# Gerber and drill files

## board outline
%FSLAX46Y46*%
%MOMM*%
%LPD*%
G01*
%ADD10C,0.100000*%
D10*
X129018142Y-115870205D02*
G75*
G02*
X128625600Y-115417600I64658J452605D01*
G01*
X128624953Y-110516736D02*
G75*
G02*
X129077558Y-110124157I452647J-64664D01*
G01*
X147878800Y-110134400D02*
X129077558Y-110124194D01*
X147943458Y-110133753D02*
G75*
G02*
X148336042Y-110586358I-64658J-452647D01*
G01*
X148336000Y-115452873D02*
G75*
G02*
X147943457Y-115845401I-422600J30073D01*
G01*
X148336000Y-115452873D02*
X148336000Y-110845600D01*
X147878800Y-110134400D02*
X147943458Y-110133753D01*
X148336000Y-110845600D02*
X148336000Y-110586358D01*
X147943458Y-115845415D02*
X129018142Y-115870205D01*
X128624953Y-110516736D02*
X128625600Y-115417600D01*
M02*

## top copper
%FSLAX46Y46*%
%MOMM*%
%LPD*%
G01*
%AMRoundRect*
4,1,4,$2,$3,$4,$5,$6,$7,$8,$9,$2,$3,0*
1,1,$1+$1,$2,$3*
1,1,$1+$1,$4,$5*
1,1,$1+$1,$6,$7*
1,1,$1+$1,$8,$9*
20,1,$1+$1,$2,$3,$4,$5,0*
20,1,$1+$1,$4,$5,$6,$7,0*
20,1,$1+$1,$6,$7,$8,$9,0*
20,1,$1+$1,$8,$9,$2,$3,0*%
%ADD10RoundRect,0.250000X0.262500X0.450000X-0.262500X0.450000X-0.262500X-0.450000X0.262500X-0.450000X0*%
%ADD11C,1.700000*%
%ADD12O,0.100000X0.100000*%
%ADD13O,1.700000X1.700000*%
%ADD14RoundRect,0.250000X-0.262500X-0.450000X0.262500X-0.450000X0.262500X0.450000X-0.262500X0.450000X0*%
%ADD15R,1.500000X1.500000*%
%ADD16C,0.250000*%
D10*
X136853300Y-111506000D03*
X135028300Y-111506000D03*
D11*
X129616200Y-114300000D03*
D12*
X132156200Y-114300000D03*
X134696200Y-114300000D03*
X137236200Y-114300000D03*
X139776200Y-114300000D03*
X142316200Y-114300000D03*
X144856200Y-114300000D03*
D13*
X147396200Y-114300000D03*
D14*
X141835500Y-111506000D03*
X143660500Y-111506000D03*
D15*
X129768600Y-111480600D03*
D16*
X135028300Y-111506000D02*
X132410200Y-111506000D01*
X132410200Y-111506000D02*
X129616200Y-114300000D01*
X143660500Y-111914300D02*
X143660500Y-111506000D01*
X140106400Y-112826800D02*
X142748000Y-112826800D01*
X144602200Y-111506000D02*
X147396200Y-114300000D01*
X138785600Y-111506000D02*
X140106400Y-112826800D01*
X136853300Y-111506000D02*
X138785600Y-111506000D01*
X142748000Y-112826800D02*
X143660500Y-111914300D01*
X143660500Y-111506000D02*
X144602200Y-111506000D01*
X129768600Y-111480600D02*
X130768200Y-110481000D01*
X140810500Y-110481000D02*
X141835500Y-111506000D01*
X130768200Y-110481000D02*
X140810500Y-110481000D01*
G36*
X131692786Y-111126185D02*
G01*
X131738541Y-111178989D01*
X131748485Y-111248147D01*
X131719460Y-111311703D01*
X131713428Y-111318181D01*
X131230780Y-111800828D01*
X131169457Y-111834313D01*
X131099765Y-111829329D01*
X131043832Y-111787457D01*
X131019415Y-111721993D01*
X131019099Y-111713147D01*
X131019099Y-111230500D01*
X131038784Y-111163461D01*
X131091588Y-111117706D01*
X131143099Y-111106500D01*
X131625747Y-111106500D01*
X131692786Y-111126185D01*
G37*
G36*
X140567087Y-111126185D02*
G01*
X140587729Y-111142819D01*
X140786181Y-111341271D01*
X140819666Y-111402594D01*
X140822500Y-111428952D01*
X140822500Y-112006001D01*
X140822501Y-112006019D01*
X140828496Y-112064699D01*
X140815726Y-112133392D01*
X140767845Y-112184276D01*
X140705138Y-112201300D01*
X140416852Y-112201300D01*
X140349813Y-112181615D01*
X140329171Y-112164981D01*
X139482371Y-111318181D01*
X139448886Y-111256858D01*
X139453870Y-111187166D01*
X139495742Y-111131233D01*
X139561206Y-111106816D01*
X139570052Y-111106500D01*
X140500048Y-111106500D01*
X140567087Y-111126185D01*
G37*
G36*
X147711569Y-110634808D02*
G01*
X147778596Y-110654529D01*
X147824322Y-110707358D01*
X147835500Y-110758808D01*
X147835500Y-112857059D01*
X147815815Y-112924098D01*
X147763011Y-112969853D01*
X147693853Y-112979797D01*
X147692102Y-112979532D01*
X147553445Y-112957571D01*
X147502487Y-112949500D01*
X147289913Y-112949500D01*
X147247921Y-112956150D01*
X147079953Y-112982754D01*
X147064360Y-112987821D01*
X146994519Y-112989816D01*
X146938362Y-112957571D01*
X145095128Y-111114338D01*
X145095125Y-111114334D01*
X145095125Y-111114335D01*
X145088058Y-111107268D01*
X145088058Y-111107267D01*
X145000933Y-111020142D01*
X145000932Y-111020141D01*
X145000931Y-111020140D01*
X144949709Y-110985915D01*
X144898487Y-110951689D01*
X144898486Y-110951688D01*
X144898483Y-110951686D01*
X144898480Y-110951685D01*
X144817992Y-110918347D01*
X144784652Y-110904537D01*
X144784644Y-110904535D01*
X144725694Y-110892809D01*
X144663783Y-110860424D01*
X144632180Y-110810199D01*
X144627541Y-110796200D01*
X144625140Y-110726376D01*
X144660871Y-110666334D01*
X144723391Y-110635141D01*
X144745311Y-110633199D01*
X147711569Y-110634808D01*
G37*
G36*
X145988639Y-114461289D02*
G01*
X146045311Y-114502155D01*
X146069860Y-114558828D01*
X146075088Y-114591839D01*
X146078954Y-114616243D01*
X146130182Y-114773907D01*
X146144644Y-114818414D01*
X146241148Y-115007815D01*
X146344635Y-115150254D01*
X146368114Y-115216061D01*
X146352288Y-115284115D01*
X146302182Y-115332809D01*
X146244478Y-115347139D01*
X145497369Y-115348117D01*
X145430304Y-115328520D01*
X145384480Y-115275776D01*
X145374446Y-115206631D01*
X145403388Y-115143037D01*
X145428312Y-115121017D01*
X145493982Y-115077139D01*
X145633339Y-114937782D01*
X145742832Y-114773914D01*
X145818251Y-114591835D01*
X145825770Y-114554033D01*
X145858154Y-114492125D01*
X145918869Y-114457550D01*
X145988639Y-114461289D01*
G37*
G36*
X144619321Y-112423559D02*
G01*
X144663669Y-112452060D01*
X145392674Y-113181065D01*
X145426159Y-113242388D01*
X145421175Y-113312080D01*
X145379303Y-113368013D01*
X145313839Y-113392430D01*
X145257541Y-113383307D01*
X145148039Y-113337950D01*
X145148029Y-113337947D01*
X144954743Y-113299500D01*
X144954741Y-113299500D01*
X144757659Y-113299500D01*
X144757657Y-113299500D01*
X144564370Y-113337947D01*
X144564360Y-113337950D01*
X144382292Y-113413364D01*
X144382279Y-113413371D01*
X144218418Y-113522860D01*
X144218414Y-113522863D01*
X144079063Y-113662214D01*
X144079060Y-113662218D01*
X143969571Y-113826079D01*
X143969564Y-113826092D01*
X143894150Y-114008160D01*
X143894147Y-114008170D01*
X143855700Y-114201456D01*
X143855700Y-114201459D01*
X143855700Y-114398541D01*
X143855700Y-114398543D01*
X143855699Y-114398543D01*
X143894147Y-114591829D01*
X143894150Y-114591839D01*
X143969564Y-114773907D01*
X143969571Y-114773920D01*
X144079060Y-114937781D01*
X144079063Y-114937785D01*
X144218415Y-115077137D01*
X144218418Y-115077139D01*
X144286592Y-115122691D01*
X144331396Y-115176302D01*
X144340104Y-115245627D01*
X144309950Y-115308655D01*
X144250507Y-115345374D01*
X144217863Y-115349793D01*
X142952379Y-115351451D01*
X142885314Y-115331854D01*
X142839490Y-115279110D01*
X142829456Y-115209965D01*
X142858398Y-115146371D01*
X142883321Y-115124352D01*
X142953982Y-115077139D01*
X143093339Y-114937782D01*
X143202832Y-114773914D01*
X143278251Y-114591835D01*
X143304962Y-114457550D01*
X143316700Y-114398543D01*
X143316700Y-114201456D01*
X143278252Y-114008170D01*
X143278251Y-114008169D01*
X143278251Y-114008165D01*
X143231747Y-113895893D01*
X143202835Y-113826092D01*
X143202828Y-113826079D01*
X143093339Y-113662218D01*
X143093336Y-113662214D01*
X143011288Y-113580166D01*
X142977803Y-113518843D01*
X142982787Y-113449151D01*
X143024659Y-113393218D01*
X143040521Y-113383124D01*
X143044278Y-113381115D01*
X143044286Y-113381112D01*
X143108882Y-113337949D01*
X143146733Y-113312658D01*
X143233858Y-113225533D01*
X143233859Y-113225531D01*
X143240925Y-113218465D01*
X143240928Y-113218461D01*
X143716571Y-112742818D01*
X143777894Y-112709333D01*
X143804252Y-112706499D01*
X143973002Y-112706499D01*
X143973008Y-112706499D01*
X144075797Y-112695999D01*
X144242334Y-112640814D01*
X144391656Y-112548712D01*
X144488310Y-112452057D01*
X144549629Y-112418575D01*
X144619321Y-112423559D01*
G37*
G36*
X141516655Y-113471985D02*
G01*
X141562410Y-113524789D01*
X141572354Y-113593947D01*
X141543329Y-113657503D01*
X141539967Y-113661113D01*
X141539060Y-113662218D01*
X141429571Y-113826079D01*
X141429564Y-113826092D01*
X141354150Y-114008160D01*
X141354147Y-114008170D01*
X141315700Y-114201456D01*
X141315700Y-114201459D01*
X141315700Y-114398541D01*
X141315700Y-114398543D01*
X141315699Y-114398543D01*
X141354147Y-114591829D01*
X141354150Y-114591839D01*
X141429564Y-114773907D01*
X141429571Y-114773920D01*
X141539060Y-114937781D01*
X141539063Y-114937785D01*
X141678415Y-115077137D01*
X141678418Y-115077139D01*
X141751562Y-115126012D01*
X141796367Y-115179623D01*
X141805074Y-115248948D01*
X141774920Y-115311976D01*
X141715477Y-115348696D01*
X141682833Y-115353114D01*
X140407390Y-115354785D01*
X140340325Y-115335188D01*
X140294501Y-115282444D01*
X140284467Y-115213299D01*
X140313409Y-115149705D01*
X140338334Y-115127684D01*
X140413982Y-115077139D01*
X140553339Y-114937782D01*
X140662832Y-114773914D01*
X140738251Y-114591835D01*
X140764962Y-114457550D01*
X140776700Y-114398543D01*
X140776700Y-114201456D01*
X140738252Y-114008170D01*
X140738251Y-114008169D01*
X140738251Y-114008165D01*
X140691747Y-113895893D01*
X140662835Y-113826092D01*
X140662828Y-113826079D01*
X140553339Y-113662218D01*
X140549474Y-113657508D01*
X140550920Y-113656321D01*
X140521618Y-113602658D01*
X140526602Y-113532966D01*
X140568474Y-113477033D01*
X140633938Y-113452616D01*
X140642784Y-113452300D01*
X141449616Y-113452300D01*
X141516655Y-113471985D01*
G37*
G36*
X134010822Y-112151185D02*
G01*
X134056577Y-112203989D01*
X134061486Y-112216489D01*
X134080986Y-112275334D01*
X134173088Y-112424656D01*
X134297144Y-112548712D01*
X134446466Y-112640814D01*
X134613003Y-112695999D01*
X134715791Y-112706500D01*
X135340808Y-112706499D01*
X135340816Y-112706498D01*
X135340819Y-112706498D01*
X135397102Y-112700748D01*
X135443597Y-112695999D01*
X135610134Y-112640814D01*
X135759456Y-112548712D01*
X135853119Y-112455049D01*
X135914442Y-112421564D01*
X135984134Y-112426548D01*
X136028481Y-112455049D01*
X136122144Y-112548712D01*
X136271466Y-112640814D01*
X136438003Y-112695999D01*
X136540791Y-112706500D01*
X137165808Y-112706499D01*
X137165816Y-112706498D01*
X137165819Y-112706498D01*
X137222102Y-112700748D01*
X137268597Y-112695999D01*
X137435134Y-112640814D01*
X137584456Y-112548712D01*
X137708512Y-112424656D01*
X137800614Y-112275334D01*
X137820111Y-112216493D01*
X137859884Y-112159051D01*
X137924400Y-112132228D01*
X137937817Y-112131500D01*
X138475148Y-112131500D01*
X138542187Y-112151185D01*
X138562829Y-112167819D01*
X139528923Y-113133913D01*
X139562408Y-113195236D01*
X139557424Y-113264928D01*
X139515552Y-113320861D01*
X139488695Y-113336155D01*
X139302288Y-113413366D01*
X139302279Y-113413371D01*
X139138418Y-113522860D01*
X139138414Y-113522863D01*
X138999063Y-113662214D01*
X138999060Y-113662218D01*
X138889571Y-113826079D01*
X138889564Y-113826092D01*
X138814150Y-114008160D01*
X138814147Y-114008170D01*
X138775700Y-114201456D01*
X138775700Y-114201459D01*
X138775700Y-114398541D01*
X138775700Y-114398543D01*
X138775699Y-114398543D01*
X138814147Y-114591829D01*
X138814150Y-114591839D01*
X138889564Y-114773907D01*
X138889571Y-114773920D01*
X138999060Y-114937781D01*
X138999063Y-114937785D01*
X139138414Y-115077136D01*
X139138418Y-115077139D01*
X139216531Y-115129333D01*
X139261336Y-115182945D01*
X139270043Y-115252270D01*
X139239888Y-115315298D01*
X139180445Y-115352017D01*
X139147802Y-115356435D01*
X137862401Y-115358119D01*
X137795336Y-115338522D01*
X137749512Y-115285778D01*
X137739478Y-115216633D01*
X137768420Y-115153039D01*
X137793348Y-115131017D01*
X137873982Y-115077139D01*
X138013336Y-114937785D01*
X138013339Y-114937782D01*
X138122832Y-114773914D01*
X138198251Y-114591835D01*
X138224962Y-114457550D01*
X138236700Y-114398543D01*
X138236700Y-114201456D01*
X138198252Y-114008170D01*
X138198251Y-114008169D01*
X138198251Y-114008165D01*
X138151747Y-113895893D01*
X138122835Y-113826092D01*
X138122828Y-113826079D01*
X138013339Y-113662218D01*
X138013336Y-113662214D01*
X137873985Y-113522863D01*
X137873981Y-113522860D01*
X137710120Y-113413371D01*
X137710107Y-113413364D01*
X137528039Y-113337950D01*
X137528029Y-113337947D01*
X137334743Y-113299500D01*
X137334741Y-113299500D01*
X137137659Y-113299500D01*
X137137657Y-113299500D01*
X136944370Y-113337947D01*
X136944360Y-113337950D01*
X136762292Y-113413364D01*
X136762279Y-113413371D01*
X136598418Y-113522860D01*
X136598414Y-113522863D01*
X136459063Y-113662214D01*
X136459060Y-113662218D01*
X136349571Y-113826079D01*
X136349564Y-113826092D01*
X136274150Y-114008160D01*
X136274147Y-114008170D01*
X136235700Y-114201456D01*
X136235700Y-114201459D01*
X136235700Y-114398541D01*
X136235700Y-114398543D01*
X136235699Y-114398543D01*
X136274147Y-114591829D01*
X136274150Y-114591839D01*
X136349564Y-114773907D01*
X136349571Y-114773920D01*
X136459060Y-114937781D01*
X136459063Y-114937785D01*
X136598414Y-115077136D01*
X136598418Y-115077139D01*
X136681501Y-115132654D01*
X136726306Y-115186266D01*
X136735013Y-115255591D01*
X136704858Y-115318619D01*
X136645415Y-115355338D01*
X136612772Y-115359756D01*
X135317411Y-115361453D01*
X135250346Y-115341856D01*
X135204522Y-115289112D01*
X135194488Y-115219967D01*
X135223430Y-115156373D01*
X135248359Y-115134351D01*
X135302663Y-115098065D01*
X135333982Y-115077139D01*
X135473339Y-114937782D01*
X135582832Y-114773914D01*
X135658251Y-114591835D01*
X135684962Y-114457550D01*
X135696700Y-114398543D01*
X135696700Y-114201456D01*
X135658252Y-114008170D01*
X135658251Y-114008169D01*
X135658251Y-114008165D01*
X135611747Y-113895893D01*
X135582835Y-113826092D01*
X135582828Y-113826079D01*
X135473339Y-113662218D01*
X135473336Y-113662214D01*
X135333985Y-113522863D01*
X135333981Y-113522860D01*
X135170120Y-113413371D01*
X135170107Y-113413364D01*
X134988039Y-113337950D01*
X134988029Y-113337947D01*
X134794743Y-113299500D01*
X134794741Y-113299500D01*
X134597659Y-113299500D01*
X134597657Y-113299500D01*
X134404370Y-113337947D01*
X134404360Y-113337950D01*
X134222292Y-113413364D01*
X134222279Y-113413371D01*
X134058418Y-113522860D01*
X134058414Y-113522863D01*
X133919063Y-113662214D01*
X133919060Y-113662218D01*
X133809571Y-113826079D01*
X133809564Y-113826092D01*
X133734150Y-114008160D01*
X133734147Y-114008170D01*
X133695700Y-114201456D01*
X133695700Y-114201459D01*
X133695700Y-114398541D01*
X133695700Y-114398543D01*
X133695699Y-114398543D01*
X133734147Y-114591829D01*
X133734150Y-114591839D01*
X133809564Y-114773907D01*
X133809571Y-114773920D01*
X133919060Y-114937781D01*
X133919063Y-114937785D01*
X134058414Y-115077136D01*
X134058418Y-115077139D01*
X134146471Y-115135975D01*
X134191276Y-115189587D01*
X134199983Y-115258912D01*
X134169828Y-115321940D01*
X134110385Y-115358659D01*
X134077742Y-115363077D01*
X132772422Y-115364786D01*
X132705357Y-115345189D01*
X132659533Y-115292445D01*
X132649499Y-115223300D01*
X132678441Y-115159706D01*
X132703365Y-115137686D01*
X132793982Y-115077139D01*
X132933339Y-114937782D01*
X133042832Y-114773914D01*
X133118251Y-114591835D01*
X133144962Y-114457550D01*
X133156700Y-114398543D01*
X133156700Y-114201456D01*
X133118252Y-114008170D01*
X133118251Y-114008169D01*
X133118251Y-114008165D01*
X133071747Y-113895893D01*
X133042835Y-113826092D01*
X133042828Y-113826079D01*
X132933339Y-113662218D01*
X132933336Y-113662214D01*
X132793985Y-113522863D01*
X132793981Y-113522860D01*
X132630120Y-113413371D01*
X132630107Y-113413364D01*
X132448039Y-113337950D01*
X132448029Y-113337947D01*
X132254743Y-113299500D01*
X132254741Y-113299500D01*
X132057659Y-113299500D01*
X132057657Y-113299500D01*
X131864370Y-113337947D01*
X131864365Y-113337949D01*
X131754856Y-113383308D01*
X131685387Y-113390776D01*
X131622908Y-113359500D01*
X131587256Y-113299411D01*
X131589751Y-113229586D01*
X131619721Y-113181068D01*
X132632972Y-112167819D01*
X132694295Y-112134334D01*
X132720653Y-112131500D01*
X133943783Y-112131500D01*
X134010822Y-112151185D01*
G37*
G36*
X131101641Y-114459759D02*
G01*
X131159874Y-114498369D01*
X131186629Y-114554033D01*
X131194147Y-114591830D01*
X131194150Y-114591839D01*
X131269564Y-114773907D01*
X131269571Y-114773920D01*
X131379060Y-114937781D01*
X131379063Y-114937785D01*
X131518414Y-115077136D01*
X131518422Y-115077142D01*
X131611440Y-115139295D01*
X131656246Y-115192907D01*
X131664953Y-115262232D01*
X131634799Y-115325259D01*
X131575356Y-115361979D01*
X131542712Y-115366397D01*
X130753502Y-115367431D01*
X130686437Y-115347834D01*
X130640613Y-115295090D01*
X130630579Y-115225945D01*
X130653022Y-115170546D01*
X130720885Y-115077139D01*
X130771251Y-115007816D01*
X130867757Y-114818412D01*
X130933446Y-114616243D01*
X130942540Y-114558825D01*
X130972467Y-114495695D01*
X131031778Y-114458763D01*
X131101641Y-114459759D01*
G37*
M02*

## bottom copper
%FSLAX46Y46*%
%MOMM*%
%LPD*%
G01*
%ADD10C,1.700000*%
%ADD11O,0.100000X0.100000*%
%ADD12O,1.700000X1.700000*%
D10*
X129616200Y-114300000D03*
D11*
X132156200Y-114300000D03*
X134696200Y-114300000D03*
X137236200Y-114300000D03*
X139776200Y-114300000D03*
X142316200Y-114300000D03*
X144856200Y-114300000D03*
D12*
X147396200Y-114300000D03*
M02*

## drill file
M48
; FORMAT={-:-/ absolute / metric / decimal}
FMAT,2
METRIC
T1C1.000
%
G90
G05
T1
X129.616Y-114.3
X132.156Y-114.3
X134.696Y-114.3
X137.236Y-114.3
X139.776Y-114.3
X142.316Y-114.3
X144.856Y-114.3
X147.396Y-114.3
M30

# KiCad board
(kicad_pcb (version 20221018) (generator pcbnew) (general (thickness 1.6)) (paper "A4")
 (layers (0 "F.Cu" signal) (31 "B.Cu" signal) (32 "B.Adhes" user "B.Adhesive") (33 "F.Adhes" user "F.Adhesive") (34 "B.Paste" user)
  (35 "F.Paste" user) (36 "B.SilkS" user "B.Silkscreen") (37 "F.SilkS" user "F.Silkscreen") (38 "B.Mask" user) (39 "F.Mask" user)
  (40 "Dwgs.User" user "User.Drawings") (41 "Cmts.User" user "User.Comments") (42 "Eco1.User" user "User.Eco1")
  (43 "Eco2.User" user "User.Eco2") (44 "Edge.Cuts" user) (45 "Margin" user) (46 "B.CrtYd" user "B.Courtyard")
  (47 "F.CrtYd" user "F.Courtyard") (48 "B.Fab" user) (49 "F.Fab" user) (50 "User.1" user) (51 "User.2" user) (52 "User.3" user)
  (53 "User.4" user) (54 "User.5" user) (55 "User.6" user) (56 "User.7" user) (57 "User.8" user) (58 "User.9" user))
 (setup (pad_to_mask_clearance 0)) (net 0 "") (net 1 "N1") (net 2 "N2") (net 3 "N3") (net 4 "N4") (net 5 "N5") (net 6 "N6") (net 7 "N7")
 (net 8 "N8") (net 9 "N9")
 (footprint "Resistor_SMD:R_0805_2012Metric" (layer "F.Cu") (at 135.9408 111.506 180)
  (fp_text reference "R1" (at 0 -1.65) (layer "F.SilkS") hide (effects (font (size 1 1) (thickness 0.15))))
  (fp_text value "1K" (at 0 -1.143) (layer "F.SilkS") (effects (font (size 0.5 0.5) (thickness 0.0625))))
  (pad "1" smd roundrect (at -0.9125 0 180) (size 1.025 1.4) (layers "F.Cu" "F.Paste" "F.Mask") (roundrect_rratio 0.243902439) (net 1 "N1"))
  (pad "2" smd roundrect (at 0.9125 0 180) (size 1.025 1.4) (layers "F.Cu" "F.Paste" "F.Mask") (roundrect_rratio 0.243902439) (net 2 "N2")))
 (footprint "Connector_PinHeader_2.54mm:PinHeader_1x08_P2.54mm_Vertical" (layer "F.Cu") (at 129.6162 114.3 90)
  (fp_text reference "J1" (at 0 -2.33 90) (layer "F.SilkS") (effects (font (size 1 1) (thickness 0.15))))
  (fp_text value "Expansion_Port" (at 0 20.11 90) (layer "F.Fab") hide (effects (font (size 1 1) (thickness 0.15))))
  (pad "1" thru_hole circle (at 0 0 90) (size 1.7 1.7) (drill 1) (layers "*.Cu" "*.Mask") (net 2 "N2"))
  (pad "2" thru_hole oval (at 0 2.54 90) (size 0.1 0.1) (drill 1) (layers "*.Cu" "*.Mask") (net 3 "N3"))
  (pad "3" thru_hole oval (at 0 5.08 90) (size 0.1 0.1) (drill 1) (layers "*.Cu" "*.Mask") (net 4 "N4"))
  (pad "4" thru_hole oval (at 0 7.62 90) (size 0.1 0.1) (drill 1) (layers "*.Cu" "*.Mask") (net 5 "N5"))
  (pad "5" thru_hole oval (at 0 10.16 90) (size 0.1 0.1) (drill 1) (layers "*.Cu" "*.Mask") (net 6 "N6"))
  (pad "6" thru_hole oval (at 0 12.7 90) (size 0.1 0.1) (drill 1) (layers "*.Cu" "*.Mask") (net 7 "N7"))
  (pad "7" thru_hole oval (at 0 15.24 90) (size 0.1 0.1) (drill 1) (layers "*.Cu" "*.Mask") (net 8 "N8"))
  (pad "8" thru_hole oval (at 0 17.78 90) (size 1.7 1.7) (drill 1) (layers "*.Cu" "*.Mask") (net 1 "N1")))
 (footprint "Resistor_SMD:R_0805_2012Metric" (layer "F.Cu") (at 142.748 111.506)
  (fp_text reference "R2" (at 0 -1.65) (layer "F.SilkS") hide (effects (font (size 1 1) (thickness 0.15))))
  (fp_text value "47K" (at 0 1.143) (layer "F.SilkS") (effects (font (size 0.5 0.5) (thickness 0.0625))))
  (pad "1" smd roundrect (at -0.9125 0) (size 1.025 1.4) (layers "F.Cu" "F.Paste" "F.Mask") (roundrect_rratio 0.243902439) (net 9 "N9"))
  (pad "2" smd roundrect (at 0.9125 0) (size 1.025 1.4) (layers "F.Cu" "F.Paste" "F.Mask") (roundrect_rratio 0.243902439) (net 1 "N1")))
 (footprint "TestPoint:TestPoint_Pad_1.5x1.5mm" (layer "F.Cu") (at 129.7686 111.4806)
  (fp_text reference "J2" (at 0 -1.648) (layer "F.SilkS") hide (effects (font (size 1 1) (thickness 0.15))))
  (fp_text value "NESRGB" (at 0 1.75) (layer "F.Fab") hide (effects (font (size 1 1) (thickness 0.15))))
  (pad "1" smd rect (at 0 0) (size 1.5 1.5) (layers "F.Cu" "F.Mask") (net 9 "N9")))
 (gr_arc (start 129.018142 115.870205) (mid 128.737407 115.717158) (end 128.6256 115.4176) (stroke (width 0.1) (type default))
  (layer "Edge.Cuts"))
 (gr_arc (start 128.624953 110.516736) (mid 128.778 110.236) (end 129.077558 110.124194) (stroke (width 0.1) (type default))
  (layer "Edge.Cuts"))
 (gr_line (start 147.8788 110.1344) (end 129.077558 110.124194) (stroke (width 0.1) (type default)) (layer "Edge.Cuts"))
 (gr_arc (start 147.943458 110.133753) (mid 148.224193 110.2868) (end 148.336 110.586358) (stroke (width 0.1) (type default))
  (layer "Edge.Cuts"))
 (gr_arc (start 148.336 115.452873) (mid 148.212985 115.7224) (end 147.943458 115.845415) (stroke (width 0.1) (type default))
  (layer "Edge.Cuts"))
 (gr_line (start 148.336 115.452873) (end 148.336 110.8456) (stroke (width 0.1) (type default)) (layer "Edge.Cuts"))
 (gr_line (start 147.8788 110.1344) (end 147.943458 110.133753) (stroke (width 0.1) (type default)) (layer "Edge.Cuts"))
 (gr_line (start 148.336 110.8456) (end 148.336 110.586358) (stroke (width 0.1) (type default)) (layer "Edge.Cuts"))
 (gr_line (start 147.943458 115.845415) (end 129.018142 115.870205) (stroke (width 0.1) (type default)) (layer "Edge.Cuts"))
 (gr_line (start 128.624953 110.516736) (end 128.6256 115.4176) (stroke (width 0.1) (type default)) (layer "Edge.Cuts"))
 (segment (start 135.0283 111.506) (end 132.4102 111.506) (width 0.25) (layer "F.Cu") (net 2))
 (segment (start 132.4102 111.506) (end 129.6162 114.3) (width 0.25) (layer "F.Cu") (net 2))
 (segment (start 143.6605 111.9143) (end 143.6605 111.506) (width 0.25) (layer "F.Cu") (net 1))
 (segment (start 140.1064 112.8268) (end 142.748 112.8268) (width 0.25) (layer "F.Cu") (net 1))
 (segment (start 144.6022 111.506) (end 147.3962 114.3) (width 0.25) (layer "F.Cu") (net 1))
 (segment (start 138.7856 111.506) (end 140.1064 112.8268) (width 0.25) (layer "F.Cu") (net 1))
 (segment (start 136.8533 111.506) (end 138.7856 111.506) (width 0.25) (layer "F.Cu") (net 1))
 (segment (start 142.748 112.8268) (end 143.6605 111.9143) (width 0.25) (layer "F.Cu") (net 1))
 (segment (start 143.6605 111.506) (end 144.6022 111.506) (width 0.25) (layer "F.Cu") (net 1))
 (segment (start 129.7686 111.4806) (end 130.7682 110.481) (width 0.25) (layer "F.Cu") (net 9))
 (segment (start 140.8105 110.481) (end 141.8355 111.506) (width 0.25) (layer "F.Cu") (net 9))
 (segment (start 130.7682 110.481) (end 140.8105 110.481) (width 0.25) (layer "F.Cu") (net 9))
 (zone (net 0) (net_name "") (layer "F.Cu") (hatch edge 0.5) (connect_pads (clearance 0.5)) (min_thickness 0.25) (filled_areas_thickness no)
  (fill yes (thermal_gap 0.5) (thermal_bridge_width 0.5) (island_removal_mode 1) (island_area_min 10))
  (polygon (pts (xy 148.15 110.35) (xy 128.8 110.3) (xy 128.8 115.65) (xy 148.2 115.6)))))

